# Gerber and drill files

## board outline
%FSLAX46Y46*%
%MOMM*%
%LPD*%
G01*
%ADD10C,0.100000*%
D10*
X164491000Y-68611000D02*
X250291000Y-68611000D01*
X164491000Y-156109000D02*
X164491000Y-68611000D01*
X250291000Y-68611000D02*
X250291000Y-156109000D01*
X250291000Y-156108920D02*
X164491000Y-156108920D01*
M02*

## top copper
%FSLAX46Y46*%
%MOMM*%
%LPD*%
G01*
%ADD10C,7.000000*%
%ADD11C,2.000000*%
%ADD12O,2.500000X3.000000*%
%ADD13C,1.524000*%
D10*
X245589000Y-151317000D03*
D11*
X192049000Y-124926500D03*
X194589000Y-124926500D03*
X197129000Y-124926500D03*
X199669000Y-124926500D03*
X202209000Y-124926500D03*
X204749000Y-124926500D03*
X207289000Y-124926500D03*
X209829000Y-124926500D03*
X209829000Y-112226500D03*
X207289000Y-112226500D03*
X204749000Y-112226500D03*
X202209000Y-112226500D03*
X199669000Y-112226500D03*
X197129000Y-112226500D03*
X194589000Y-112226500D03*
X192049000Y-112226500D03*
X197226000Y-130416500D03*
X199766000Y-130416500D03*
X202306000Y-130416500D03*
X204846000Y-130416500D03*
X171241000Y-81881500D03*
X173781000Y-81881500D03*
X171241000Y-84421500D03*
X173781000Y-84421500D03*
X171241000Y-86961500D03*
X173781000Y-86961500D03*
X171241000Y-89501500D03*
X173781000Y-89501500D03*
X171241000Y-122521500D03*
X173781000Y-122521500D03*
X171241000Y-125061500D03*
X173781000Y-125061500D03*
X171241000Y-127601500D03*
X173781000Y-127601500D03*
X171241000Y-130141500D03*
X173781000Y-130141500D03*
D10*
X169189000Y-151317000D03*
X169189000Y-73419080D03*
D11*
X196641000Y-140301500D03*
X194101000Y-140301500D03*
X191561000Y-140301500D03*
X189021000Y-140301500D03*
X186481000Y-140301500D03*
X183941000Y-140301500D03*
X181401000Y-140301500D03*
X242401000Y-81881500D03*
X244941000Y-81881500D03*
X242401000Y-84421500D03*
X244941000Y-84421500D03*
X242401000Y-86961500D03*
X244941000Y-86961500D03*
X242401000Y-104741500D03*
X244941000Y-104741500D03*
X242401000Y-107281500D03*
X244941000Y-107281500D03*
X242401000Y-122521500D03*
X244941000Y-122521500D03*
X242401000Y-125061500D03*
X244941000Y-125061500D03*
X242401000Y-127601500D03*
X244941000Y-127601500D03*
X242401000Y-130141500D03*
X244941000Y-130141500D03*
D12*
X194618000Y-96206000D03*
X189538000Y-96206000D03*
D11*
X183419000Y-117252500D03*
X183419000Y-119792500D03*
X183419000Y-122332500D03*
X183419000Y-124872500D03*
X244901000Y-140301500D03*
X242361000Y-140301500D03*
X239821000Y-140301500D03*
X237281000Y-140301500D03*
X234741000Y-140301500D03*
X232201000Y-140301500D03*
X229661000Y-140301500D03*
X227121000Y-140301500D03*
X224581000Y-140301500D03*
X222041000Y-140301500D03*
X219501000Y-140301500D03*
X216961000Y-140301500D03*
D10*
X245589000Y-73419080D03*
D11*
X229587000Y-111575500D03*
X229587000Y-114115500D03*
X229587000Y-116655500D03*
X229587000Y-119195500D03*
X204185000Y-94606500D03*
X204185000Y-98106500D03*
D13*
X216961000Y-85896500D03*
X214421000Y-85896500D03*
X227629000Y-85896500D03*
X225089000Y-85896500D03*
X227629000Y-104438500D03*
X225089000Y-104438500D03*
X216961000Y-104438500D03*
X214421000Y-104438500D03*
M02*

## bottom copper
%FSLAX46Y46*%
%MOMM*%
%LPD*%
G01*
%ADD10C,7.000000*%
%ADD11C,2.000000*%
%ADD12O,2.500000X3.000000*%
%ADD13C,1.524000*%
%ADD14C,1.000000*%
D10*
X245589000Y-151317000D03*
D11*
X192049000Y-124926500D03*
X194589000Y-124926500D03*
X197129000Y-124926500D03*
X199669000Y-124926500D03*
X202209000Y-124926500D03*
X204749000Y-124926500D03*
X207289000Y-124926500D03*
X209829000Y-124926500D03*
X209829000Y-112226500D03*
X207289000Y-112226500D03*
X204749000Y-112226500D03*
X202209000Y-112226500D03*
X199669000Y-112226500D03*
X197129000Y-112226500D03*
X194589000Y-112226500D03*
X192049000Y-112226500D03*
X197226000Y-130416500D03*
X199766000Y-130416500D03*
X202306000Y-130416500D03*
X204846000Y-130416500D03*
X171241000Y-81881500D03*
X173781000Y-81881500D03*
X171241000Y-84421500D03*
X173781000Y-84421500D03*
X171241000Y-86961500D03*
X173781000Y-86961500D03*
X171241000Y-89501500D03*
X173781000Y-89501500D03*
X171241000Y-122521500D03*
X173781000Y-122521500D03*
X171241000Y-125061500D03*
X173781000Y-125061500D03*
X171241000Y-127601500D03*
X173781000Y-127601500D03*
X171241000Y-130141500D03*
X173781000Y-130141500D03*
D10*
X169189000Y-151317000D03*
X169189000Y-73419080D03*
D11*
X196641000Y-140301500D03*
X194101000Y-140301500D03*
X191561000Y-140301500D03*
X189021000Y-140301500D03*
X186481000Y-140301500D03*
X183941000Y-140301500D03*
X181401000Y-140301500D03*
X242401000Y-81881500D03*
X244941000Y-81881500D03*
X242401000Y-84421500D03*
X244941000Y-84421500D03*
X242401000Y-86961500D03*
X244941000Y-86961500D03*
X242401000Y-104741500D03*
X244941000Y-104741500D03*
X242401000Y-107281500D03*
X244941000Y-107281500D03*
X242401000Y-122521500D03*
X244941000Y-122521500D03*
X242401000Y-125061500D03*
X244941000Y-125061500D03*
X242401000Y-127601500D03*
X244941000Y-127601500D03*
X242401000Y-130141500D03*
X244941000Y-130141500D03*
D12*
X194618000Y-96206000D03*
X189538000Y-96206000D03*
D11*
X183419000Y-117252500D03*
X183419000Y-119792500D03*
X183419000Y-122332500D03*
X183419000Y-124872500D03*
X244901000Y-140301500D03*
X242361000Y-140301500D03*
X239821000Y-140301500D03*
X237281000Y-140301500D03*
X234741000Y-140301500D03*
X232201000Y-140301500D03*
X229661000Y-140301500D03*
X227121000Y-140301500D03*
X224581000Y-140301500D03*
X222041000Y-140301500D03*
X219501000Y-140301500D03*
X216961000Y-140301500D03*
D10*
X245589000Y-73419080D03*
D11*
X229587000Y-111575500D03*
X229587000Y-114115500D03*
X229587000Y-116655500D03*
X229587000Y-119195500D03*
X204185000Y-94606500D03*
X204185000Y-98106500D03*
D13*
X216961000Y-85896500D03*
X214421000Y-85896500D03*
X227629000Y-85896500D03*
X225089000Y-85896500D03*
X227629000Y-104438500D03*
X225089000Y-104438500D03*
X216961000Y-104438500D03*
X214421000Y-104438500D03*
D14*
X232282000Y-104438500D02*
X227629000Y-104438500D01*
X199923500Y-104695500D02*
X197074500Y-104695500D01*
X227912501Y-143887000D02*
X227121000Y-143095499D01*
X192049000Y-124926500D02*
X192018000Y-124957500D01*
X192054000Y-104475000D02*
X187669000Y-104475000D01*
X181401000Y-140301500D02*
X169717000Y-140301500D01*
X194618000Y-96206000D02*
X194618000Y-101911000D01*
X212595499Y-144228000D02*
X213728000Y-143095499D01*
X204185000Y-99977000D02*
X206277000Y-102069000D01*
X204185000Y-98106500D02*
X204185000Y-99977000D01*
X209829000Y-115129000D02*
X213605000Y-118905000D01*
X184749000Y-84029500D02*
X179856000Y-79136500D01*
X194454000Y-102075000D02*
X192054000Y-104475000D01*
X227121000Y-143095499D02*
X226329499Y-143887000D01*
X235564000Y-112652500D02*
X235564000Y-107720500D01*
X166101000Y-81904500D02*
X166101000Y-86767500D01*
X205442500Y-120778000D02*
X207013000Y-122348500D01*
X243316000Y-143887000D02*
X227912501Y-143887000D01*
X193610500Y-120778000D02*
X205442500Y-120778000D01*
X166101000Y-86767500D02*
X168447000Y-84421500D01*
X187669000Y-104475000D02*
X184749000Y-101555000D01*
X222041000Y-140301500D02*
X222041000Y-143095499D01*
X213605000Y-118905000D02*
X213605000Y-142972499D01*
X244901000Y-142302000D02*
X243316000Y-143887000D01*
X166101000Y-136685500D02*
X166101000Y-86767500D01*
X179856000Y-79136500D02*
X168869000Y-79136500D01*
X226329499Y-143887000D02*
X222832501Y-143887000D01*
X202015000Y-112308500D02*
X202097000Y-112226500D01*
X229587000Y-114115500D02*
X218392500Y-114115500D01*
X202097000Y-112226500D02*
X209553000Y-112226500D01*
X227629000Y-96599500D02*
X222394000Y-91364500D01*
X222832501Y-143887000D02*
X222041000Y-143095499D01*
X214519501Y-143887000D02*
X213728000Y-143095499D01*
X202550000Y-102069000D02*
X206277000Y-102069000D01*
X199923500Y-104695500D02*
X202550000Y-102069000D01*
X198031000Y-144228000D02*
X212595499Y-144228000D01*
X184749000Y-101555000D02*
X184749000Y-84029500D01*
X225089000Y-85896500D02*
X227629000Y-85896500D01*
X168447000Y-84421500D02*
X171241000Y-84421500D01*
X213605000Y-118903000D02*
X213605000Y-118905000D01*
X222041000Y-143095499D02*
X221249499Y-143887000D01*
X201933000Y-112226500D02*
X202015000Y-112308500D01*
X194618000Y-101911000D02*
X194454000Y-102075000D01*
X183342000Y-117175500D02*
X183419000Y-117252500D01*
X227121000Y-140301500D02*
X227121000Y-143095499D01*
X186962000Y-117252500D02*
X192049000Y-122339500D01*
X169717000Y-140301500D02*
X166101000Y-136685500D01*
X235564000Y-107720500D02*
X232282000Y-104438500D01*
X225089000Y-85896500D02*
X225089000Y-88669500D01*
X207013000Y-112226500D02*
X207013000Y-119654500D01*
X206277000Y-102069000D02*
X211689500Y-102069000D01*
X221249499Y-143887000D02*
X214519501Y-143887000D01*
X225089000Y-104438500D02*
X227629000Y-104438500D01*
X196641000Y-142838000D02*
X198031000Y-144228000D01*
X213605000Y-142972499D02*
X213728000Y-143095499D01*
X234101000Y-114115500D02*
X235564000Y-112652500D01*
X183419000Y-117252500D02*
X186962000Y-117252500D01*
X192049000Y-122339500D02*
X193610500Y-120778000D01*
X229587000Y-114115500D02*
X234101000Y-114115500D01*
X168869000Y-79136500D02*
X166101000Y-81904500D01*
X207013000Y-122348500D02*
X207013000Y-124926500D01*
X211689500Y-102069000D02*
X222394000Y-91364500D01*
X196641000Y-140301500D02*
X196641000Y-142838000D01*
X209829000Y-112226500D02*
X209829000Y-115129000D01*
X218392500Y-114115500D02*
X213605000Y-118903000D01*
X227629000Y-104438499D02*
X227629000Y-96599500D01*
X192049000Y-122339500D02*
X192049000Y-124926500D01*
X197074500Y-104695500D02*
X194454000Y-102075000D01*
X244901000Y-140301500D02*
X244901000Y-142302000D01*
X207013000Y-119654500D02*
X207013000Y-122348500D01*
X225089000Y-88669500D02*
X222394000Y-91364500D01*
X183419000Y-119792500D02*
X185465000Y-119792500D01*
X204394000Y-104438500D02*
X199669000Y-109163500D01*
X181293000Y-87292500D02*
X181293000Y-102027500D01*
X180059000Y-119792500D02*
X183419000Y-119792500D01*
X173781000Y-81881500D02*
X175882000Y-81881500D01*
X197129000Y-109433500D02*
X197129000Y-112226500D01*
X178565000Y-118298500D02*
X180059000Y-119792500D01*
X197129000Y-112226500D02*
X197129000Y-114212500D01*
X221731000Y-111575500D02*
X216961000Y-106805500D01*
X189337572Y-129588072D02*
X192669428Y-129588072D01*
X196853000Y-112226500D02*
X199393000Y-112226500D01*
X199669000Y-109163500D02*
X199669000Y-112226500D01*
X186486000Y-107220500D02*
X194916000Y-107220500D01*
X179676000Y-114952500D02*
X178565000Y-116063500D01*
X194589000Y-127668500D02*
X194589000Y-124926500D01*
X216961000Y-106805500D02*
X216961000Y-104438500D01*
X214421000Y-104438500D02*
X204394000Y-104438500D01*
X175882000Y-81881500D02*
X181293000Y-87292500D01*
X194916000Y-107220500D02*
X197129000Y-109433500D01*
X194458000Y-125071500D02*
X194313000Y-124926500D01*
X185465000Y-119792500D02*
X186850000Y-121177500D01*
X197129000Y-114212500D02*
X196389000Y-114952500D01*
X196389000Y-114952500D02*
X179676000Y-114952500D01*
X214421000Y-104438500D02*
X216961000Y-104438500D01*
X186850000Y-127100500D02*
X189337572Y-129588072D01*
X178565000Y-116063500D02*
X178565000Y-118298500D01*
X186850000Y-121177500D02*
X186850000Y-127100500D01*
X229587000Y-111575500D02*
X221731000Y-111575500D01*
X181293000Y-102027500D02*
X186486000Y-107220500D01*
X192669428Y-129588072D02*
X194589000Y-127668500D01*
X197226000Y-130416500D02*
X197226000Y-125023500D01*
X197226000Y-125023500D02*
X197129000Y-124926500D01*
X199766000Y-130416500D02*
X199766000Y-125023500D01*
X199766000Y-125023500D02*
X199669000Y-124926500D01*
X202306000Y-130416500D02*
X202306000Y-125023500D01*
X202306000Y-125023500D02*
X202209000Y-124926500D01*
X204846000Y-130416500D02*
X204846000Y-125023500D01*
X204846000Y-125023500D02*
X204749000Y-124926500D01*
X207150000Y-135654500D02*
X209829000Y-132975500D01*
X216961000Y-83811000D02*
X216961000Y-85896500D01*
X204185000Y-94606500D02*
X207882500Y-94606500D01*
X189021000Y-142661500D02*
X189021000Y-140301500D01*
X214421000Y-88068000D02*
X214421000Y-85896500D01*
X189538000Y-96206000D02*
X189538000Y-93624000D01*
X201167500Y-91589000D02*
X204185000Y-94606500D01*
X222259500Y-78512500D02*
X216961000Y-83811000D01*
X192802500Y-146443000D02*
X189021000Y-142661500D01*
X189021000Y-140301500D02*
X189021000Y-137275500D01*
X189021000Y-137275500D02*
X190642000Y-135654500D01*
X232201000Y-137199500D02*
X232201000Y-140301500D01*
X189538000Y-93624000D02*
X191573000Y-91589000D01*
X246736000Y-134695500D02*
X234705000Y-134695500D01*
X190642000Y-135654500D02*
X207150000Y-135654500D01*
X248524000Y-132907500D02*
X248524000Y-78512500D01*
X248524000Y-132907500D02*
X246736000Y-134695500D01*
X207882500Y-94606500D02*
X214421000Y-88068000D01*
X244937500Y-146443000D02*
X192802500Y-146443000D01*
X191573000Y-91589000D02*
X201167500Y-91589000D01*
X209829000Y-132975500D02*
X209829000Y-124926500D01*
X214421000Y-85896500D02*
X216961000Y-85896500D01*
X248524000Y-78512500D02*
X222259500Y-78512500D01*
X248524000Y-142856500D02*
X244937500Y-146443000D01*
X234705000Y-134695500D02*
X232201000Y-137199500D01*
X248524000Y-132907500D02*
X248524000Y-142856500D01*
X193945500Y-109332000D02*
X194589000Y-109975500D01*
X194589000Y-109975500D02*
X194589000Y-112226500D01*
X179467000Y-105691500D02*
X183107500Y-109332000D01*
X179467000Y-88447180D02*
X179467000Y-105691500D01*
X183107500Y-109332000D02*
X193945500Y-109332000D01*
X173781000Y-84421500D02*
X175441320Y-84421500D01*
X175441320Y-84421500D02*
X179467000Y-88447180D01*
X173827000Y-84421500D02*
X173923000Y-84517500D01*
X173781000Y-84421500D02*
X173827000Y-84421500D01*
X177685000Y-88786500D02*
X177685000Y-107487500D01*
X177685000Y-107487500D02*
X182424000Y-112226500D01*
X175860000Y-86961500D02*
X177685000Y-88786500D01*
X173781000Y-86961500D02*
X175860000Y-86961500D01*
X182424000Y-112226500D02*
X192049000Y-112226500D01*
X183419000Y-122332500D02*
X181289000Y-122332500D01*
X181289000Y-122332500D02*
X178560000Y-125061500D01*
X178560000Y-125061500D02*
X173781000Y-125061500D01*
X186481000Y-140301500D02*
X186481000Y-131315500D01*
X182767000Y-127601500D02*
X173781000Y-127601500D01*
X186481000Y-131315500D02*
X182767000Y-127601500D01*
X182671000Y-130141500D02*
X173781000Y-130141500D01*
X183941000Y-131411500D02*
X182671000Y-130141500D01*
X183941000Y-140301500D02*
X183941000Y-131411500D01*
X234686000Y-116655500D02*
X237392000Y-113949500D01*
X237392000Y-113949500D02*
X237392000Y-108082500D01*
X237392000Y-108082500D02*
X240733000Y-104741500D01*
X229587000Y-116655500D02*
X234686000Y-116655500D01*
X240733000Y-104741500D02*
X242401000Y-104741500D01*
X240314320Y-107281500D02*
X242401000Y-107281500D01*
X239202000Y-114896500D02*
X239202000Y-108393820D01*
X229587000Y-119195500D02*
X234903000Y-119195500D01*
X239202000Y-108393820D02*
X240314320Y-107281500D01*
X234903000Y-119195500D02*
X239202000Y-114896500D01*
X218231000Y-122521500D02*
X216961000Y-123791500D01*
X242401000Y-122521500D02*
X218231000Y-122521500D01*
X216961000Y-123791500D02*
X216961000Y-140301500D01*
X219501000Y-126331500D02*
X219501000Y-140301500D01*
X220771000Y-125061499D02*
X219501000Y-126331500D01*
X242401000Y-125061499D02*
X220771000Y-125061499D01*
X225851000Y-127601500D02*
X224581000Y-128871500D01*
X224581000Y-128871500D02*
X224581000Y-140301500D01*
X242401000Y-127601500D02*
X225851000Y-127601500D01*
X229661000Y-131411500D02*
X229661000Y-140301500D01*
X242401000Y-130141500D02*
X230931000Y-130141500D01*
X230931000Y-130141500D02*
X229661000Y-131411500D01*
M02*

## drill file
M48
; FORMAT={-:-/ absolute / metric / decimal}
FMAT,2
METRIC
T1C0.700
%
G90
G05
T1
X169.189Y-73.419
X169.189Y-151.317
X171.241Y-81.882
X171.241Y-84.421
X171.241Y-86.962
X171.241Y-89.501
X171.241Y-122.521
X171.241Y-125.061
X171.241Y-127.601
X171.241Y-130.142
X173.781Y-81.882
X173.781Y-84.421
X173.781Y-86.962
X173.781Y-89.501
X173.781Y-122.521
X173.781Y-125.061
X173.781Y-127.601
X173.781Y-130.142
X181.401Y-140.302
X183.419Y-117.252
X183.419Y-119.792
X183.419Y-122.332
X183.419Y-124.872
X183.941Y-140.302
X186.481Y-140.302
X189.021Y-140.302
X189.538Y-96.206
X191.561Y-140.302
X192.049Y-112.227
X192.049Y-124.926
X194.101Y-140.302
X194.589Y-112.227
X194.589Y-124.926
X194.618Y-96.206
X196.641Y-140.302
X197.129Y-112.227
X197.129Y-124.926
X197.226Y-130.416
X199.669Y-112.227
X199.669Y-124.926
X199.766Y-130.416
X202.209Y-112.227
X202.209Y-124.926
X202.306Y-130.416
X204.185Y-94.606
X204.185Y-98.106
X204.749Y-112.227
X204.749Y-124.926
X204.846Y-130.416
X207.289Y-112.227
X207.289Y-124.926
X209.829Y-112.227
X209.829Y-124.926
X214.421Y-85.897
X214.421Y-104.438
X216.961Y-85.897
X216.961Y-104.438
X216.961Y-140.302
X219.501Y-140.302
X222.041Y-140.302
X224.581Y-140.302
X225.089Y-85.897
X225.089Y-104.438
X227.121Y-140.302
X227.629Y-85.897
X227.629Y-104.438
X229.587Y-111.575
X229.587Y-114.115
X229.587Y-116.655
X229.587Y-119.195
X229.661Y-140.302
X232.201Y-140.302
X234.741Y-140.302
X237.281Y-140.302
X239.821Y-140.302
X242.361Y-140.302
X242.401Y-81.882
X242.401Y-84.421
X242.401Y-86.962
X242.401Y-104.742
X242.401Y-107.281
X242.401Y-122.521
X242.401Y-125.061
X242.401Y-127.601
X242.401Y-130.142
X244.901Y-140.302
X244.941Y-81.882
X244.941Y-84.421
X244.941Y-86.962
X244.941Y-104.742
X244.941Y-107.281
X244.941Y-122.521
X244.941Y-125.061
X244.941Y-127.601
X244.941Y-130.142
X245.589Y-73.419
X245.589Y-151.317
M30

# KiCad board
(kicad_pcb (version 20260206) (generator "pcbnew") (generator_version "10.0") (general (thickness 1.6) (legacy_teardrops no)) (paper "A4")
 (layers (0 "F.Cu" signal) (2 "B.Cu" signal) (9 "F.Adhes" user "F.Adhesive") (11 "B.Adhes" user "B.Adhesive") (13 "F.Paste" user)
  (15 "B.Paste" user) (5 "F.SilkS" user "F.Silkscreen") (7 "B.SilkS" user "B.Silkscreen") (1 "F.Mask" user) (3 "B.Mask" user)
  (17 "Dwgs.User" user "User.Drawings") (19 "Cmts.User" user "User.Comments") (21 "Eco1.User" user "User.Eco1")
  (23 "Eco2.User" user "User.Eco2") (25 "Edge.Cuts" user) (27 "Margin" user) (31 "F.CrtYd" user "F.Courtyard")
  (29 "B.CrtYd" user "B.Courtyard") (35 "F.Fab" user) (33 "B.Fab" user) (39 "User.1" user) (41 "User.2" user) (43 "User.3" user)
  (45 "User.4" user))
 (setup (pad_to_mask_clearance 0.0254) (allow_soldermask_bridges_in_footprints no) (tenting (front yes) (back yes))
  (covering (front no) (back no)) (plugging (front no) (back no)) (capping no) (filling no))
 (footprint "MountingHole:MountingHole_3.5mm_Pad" (layer "F.Cu") (at 245.589 151.317)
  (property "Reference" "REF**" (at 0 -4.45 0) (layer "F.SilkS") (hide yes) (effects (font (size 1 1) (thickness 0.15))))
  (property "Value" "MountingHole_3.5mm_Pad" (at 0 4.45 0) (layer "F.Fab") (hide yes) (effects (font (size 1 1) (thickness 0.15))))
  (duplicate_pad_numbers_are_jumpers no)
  (pad "1" thru_hole circle (at 0 0) (size 7 7) (drill 0.7) (layers "*.Cu" "*.Mask") (remove_unused_layers no) (zone_connect 2)))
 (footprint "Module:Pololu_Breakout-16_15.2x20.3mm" (layer "F.Cu") (at 192.049 124.9265 90)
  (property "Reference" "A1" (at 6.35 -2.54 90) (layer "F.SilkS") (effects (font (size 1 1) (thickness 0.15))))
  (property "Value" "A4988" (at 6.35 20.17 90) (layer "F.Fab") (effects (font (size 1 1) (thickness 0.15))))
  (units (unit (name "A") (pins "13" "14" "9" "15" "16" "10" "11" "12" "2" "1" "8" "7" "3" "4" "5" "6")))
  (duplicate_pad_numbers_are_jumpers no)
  (pad "1" thru_hole circle (at 0 0 90) (size 2 2) (drill 0.7) (layers "*.Cu" "*.Mask") (remove_unused_layers no) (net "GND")
   (thermal_bridge_angle 90))
  (pad "2" thru_hole circle (at 0 2.54 90) (size 2 2) (drill 0.7) (layers "*.Cu" "*.Mask") (remove_unused_layers no) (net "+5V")
   (thermal_bridge_angle 90))
  (pad "3" thru_hole circle (at 0 5.08 90) (size 2 2) (drill 0.7) (layers "*.Cu" "*.Mask") (remove_unused_layers no) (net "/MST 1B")
   (thermal_bridge_angle 90))
  (pad "4" thru_hole circle (at 0 7.62 90) (size 2 2) (drill 0.7) (layers "*.Cu" "*.Mask") (remove_unused_layers no) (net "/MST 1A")
   (thermal_bridge_angle 90))
  (pad "5" thru_hole circle (at 0 10.16 90) (size 2 2) (drill 0.7) (layers "*.Cu" "*.Mask") (remove_unused_layers no) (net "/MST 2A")
   (thermal_bridge_angle 90))
  (pad "6" thru_hole circle (at 0 12.7 90) (size 2 2) (drill 0.7) (layers "*.Cu" "*.Mask") (remove_unused_layers no) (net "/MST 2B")
   (thermal_bridge_angle 90))
  (pad "7" thru_hole circle (at 0 15.24 90) (size 2 2) (drill 0.7) (layers "*.Cu" "*.Mask") (remove_unused_layers no) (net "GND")
   (thermal_bridge_angle 90))
  (pad "8" thru_hole circle (at 0 17.78 90) (size 2 2) (drill 0.7) (layers "*.Cu" "*.Mask") (remove_unused_layers no) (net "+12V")
   (thermal_bridge_angle 90))
  (pad "9" thru_hole circle (at 12.7 17.78 90) (size 2 2) (drill 0.7) (layers "*.Cu" "*.Mask") (remove_unused_layers no) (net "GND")
   (thermal_bridge_angle 90))
  (pad "10" thru_hole circle (at 12.7 15.24 90) (size 2 2) (drill 0.7) (layers "*.Cu" "*.Mask") (remove_unused_layers no) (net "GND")
   (thermal_bridge_angle 90))
  (pad "11" thru_hole circle (at 12.7 12.7 90) (size 2 2) (drill 0.7) (layers "*.Cu" "*.Mask") (remove_unused_layers no) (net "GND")
   (thermal_bridge_angle 90))
  (pad "12" thru_hole circle (at 12.7 10.16 90) (size 2 2) (drill 0.7) (layers "*.Cu" "*.Mask") (remove_unused_layers no) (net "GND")
   (thermal_bridge_angle 90))
  (pad "13" thru_hole circle (at 12.7 7.62 90) (size 2 2) (drill 0.7) (layers "*.Cu" "*.Mask") (remove_unused_layers no) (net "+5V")
   (thermal_bridge_angle 90))
  (pad "14" thru_hole circle (at 12.7 5.08 90) (size 2 2) (drill 0.7) (layers "*.Cu" "*.Mask") (remove_unused_layers no) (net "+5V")
   (thermal_bridge_angle 90))
  (pad "15" thru_hole circle (at 12.7 2.54 90) (size 2 2) (drill 0.7) (layers "*.Cu" "*.Mask") (remove_unused_layers no) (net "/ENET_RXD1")
   (thermal_bridge_angle 90))
  (pad "16" thru_hole circle (at 12.7 0 90) (size 2 2) (drill 0.7) (layers "*.Cu" "*.Mask") (remove_unused_layers no) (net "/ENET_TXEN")
   (thermal_bridge_angle 90)))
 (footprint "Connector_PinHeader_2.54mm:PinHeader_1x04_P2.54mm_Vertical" (layer "F.Cu") (at 197.226 130.4165 90)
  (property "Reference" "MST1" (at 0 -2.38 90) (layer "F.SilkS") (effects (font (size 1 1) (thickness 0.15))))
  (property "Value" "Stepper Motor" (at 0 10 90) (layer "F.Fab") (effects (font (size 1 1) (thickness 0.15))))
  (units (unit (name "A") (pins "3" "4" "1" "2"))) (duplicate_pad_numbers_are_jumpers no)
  (pad "1" thru_hole circle (at 0 0 90) (size 2 2) (drill 0.7) (layers "*.Cu" "*.Mask") (remove_unused_layers no) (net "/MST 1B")
   (thermal_bridge_angle 90))
  (pad "2" thru_hole circle (at 0 2.54 90) (size 2 2) (drill 0.7) (layers "*.Cu" "*.Mask") (remove_unused_layers no) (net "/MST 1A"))
  (pad "3" thru_hole circle (at 0 5.08 90) (size 2 2) (drill 0.7) (layers "*.Cu" "*.Mask") (remove_unused_layers no) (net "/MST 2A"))
  (pad "4" thru_hole circle (at 0 7.62 90) (size 2 2) (drill 0.7) (layers "*.Cu" "*.Mask") (remove_unused_layers no) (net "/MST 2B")))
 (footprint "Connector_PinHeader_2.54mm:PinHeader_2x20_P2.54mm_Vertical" (layer "F.Cu") (at 171.241 81.8815)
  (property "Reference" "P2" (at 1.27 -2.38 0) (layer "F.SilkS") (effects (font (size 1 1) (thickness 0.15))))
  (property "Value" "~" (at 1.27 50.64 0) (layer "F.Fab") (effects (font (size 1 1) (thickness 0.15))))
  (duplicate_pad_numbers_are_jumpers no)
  (pad "1" thru_hole circle (at 0 0) (size 2 2) (drill 0.7) (layers "*.Cu" "*.Mask") (remove_unused_layers no)
   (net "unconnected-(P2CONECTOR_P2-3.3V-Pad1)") (thermal_bridge_angle 90))
  (pad "2" thru_hole circle (at 2.54 0) (size 2 2) (drill 0.7) (layers "*.Cu" "*.Mask") (remove_unused_layers no) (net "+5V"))
  (pad "3" thru_hole circle (at 0 2.54) (size 2 2) (drill 0.7) (layers "*.Cu" "*.Mask") (remove_unused_layers no) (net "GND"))
  (pad "4" thru_hole circle (at 2.54 2.54) (size 2 2) (drill 0.7) (layers "*.Cu" "*.Mask") (remove_unused_layers no) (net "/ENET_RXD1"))
  (pad "5" thru_hole circle (at 0 5.08) (size 2 2) (drill 0.7) (layers "*.Cu" "*.Mask") (remove_unused_layers no)
   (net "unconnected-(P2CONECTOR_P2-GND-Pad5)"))
  (pad "6" thru_hole circle (at 2.54 5.08) (size 2 2) (drill 0.7) (layers "*.Cu" "*.Mask") (remove_unused_layers no) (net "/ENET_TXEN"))
  (pad "7" thru_hole circle (at 0 7.62) (size 2 2) (drill 0.7) (layers "*.Cu" "*.Mask") (remove_unused_layers no)
   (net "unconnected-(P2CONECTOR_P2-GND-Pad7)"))
  (pad "8" thru_hole circle (at 2.54 7.62) (size 2 2) (drill 0.7) (layers "*.Cu" "*.Mask") (remove_unused_layers no)
   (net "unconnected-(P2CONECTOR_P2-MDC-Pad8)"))
  (pad "33" thru_hole circle (at 0 40.64) (size 2 2) (drill 0.7) (layers "*.Cu" "*.Mask") (remove_unused_layers no)
   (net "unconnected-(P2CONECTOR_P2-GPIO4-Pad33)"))
  (pad "34" thru_hole circle (at 2.54 40.64) (size 2 2) (drill 0.7) (layers "*.Cu" "*.Mask") (remove_unused_layers no)
   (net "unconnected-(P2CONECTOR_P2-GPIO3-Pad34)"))
  (pad "35" thru_hole circle (at 0 43.18) (size 2 2) (drill 0.7) (layers "*.Cu" "*.Mask") (remove_unused_layers no)
   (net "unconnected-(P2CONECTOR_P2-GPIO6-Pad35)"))
  (pad "36" thru_hole circle (at 2.54 43.18) (size 2 2) (drill 0.7) (layers "*.Cu" "*.Mask") (remove_unused_layers no) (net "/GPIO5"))
  (pad "37" thru_hole circle (at 0 45.72) (size 2 2) (drill 0.7) (layers "*.Cu" "*.Mask") (remove_unused_layers no)
   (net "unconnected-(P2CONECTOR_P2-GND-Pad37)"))
  (pad "38" thru_hole circle (at 2.54 45.72) (size 2 2) (drill 0.7) (layers "*.Cu" "*.Mask") (remove_unused_layers no) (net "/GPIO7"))
  (pad "39" thru_hole circle (at 0 48.26) (size 2 2) (drill 0.7) (layers "*.Cu" "*.Mask") (remove_unused_layers no)
   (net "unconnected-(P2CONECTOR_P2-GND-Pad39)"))
  (pad "40" thru_hole circle (at 2.54 48.26) (size 2 2) (drill 0.7) (layers "*.Cu" "*.Mask") (remove_unused_layers no) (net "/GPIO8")))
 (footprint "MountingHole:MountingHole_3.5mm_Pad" (layer "F.Cu") (at 169.189 151.317)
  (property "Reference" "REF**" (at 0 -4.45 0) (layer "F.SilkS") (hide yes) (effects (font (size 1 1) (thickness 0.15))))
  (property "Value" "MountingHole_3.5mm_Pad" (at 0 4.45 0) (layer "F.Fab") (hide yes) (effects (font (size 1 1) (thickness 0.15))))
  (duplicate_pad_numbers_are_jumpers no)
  (pad "1" thru_hole circle (at 0 0) (size 7 7) (drill 0.7) (layers "*.Cu" "*.Mask") (remove_unused_layers no) (zone_connect 2)))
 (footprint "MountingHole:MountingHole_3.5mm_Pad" (layer "F.Cu") (at 169.189 73.41908)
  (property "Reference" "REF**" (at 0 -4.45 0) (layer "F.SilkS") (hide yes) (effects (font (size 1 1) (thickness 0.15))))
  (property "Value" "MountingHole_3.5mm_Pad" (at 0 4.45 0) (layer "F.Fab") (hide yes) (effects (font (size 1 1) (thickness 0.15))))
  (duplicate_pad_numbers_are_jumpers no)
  (pad "1" thru_hole circle (at 0 0) (size 7 7) (drill 0.7) (layers "*.Cu" "*.Mask") (remove_unused_layers no) (zone_connect 2)))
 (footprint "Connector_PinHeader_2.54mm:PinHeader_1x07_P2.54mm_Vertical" (layer "F.Cu") (at 196.641 140.3015 -90)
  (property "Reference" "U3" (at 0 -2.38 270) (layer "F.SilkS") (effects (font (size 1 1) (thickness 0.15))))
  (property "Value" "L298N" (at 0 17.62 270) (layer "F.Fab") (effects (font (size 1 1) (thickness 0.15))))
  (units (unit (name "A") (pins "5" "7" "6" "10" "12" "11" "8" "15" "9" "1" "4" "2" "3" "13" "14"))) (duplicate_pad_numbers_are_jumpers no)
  (pad "1" thru_hole circle (at 0 0 270) (size 2 2) (drill 0.7) (layers "*.Cu" "*.Mask") (remove_unused_layers no) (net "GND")
   (thermal_bridge_angle 90))
  (pad "2" thru_hole circle (at 0 2.54 270) (size 2 2) (drill 0.7) (layers "*.Cu" "*.Mask") (remove_unused_layers no) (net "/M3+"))
  (pad "3" thru_hole circle (at 0 5.08 270) (size 2 2) (drill 0.7) (layers "*.Cu" "*.Mask") (remove_unused_layers no) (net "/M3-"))
  (pad "4" thru_hole circle (at 0 7.62 270) (size 2 2) (drill 0.7) (layers "*.Cu" "*.Mask") (remove_unused_layers no) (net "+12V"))
  (pad "5" thru_hole circle (at 0 10.16 270) (size 2 2) (drill 0.7) (layers "*.Cu" "*.Mask") (remove_unused_layers no) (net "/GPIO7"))
  (pad "6" thru_hole circle (at 0 12.7 270) (size 2 2) (drill 0.7) (layers "*.Cu" "*.Mask") (remove_unused_layers no) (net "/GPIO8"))
  (pad "7" thru_hole circle (at 0 15.24 270) (size 2 2) (drill 0.7) (layers "*.Cu" "*.Mask") (remove_unused_layers no) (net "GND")))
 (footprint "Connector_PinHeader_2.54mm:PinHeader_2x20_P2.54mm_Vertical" (layer "F.Cu") (at 242.401 81.8815)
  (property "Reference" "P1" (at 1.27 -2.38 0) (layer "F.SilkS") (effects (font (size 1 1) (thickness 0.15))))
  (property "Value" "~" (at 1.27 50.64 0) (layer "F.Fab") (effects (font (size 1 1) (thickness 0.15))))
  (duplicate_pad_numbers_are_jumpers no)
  (pad "1" thru_hole circle (at 0 0) (size 2 2) (drill 0.7) (layers "*.Cu" "*.Mask") (remove_unused_layers no)
   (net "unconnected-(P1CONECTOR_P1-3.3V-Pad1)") (thermal_bridge_angle 90))
  (pad "2" thru_hole circle (at 2.54 0) (size 2 2) (drill 0.7) (layers "*.Cu" "*.Mask") (remove_unused_layers no)
   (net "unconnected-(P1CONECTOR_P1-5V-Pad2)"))
  (pad "3" thru_hole circle (at 0 2.54) (size 2 2) (drill 0.7) (layers "*.Cu" "*.Mask") (remove_unused_layers no)
   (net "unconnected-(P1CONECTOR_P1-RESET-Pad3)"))
  (pad "4" thru_hole circle (at 2.54 2.54) (size 2 2) (drill 0.7) (layers "*.Cu" "*.Mask") (remove_unused_layers no)
   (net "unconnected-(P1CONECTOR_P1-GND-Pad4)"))
  (pad "5" thru_hole circle (at 0 5.08) (size 2 2) (drill 0.7) (layers "*.Cu" "*.Mask") (remove_unused_layers no)
   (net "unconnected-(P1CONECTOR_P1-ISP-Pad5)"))
  (pad "6" thru_hole circle (at 2.54 5.08) (size 2 2) (drill 0.7) (layers "*.Cu" "*.Mask") (remove_unused_layers no)
   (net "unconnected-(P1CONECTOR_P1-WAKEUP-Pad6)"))
  (pad "19" thru_hole circle (at 0 22.86) (size 2 2) (drill 0.7) (layers "*.Cu" "*.Mask") (remove_unused_layers no) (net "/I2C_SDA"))
  (pad "20" thru_hole circle (at 2.54 22.86) (size 2 2) (drill 0.7) (layers "*.Cu" "*.Mask") (remove_unused_layers no)
   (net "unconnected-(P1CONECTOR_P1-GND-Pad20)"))
  (pad "21" thru_hole circle (at 0 25.4) (size 2 2) (drill 0.7) (layers "*.Cu" "*.Mask") (remove_unused_layers no) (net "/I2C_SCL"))
  (pad "22" thru_hole circle (at 2.54 25.4) (size 2 2) (drill 0.7) (layers "*.Cu" "*.Mask") (remove_unused_layers no)
   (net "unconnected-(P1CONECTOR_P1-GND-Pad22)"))
  (pad "33" thru_hole circle (at 0 40.64) (size 2 2) (drill 0.7) (layers "*.Cu" "*.Mask") (remove_unused_layers no) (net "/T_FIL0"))
  (pad "34" thru_hole circle (at 2.54 40.64) (size 2 2) (drill 0.7) (layers "*.Cu" "*.Mask") (remove_unused_layers no)
   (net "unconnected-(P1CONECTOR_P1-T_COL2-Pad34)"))
  (pad "35" thru_hole circle (at 0 43.18) (size 2 2) (drill 0.7) (layers "*.Cu" "*.Mask") (remove_unused_layers no) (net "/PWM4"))
  (pad "36" thru_hole circle (at 2.54 43.18) (size 2 2) (drill 0.7) (layers "*.Cu" "*.Mask") (remove_unused_layers no)
   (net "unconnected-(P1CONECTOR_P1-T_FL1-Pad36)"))
  (pad "37" thru_hole circle (at 0 45.72) (size 2 2) (drill 0.7) (layers "*.Cu" "*.Mask") (remove_unused_layers no) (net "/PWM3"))
  (pad "38" thru_hole circle (at 2.54 45.72) (size 2 2) (drill 0.7) (layers "*.Cu" "*.Mask") (remove_unused_layers no)
   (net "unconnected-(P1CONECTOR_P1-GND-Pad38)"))
  (pad "39" thru_hole circle (at 0 48.26) (size 2 2) (drill 0.7) (layers "*.Cu" "*.Mask") (remove_unused_layers no) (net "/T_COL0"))
  (pad "40" thru_hole circle (at 2.54 48.26) (size 2 2) (drill 0.7) (layers "*.Cu" "*.Mask") (remove_unused_layers no)
   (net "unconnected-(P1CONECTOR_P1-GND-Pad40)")))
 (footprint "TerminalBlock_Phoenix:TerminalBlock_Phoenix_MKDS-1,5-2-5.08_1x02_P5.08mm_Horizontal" (layer "F.Cu") (at 194.618 96.206 180)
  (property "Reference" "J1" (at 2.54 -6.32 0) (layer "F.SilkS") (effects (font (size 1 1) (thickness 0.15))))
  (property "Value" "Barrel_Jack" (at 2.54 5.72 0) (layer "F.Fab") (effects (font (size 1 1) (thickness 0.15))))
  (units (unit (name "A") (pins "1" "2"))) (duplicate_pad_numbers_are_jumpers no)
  (pad "1" thru_hole oval (at 0 0 180) (size 2.5 3) (drill 0.7) (layers "*.Cu" "*.Mask") (remove_unused_layers no) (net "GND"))
  (pad "2" thru_hole oval (at 5.08 0 180) (size 2.5 3) (drill 0.7) (layers "*.Cu" "*.Mask") (remove_unused_layers no) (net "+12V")
   (thermal_bridge_angle 45)))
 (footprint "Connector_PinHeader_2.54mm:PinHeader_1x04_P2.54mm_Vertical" (layer "F.Cu") (at 183.419 117.2525)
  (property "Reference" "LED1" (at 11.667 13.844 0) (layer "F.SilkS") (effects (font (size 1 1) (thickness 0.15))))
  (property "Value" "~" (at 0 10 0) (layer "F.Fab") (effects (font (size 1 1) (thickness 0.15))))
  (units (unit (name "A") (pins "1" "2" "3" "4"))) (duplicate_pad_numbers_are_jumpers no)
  (pad "1" thru_hole circle (at 0 0) (size 2 2) (drill 0.7) (layers "*.Cu" "*.Mask") (remove_unused_layers no) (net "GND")
   (thermal_bridge_angle 90))
  (pad "2" thru_hole circle (at 0 2.54) (size 2 2) (drill 0.7) (layers "*.Cu" "*.Mask") (remove_unused_layers no) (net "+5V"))
  (pad "3" thru_hole circle (at 0 5.08) (size 2 2) (drill 0.7) (layers "*.Cu" "*.Mask") (remove_unused_layers no) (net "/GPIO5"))
  (pad "4" thru_hole circle (at 0 7.62) (size 2 2) (drill 0.7) (layers "*.Cu" "*.Mask") (remove_unused_layers no)
   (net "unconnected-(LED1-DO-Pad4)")))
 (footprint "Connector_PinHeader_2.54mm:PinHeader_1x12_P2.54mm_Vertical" (layer "F.Cu") (at 244.901 140.3015 -90)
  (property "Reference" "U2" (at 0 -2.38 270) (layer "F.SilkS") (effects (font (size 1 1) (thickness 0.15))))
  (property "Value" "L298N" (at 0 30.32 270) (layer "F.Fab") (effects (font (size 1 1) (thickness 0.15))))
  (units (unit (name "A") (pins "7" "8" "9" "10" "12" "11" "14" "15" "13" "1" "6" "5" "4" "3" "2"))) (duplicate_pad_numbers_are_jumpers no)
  (pad "1" thru_hole circle (at 0 0 270) (size 2 2) (drill 0.7) (layers "*.Cu" "*.Mask") (remove_unused_layers no) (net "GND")
   (thermal_bridge_angle 90))
  (pad "2" thru_hole circle (at 0 2.54 270) (size 2 2) (drill 0.7) (layers "*.Cu" "*.Mask") (remove_unused_layers no) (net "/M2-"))
  (pad "3" thru_hole circle (at 0 5.08 270) (size 2 2) (drill 0.7) (layers "*.Cu" "*.Mask") (remove_unused_layers no) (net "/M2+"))
  (pad "4" thru_hole circle (at 0 7.62 270) (size 2 2) (drill 0.7) (layers "*.Cu" "*.Mask") (remove_unused_layers no) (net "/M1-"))
  (pad "5" thru_hole circle (at 0 10.16 270) (size 2 2) (drill 0.7) (layers "*.Cu" "*.Mask") (remove_unused_layers no) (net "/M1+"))
  (pad "6" thru_hole circle (at 0 12.7 270) (size 2 2) (drill 0.7) (layers "*.Cu" "*.Mask") (remove_unused_layers no) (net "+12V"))
  (pad "7" thru_hole circle (at 0 15.24 270) (size 2 2) (drill 0.7) (layers "*.Cu" "*.Mask") (remove_unused_layers no) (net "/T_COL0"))
  (pad "8" thru_hole circle (at 0 17.78 270) (size 2 2) (drill 0.7) (layers "*.Cu" "*.Mask") (remove_unused_layers no) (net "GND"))
  (pad "9" thru_hole circle (at 0 20.32 270) (size 2 2) (drill 0.7) (layers "*.Cu" "*.Mask") (remove_unused_layers no) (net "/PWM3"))
  (pad "10" thru_hole circle (at 0 22.86 270) (size 2 2) (drill 0.7) (layers "*.Cu" "*.Mask") (remove_unused_layers no) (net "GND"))
  (pad "11" thru_hole circle (at 0 25.4 270) (size 2 2) (drill 0.7) (layers "*.Cu" "*.Mask") (remove_unused_layers no) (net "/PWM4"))
  (pad "12" thru_hole circle (at 0 27.94 270) (size 2 2) (drill 0.7) (layers "*.Cu" "*.Mask") (remove_unused_layers no) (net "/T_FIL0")))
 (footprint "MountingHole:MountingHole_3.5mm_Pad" (layer "F.Cu") (at 245.589 73.41908)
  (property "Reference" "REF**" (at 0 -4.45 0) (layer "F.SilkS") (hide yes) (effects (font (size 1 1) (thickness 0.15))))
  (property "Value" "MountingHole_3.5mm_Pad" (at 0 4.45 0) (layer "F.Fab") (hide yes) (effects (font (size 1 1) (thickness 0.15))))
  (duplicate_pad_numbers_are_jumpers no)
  (pad "1" thru_hole circle (at 0 0) (size 7 7) (drill 0.7) (layers "*.Cu" "*.Mask") (remove_unused_layers no) (zone_connect 2)))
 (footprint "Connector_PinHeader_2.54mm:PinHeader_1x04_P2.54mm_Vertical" (layer "F.Cu") (at 229.587 111.5755)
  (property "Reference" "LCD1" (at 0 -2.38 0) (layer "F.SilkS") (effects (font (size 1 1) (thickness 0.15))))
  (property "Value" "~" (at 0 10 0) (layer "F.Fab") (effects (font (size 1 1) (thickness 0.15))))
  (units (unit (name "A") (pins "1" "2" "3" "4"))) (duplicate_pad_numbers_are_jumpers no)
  (pad "1" thru_hole circle (at 0 0) (size 2 2) (drill 0.7) (layers "*.Cu" "*.Mask") (remove_unused_layers no) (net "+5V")
   (thermal_bridge_angle 90))
  (pad "2" thru_hole circle (at 0 2.54) (size 2 2) (drill 0.7) (layers "*.Cu" "*.Mask") (remove_unused_layers no) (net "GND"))
  (pad "3" thru_hole circle (at 0 5.08) (size 2 2) (drill 0.7) (layers "*.Cu" "*.Mask") (remove_unused_layers no) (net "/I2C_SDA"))
  (pad "4" thru_hole circle (at 0 7.62) (size 2 2) (drill 0.7) (layers "*.Cu" "*.Mask") (remove_unused_layers no) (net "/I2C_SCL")))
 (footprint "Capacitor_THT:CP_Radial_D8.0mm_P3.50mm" (layer "F.Cu") (at 204.185 94.6065 -90)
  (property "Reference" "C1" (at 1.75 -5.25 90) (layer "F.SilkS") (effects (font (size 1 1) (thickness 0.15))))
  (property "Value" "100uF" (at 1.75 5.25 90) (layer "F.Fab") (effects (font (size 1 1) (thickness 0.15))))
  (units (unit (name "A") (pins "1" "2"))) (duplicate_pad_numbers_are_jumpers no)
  (pad "1" thru_hole circle (at 0 0 270) (size 2 2) (drill 0.7) (layers "*.Cu" "*.Mask") (remove_unused_layers no) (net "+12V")
   (thermal_bridge_angle 90))
  (pad "2" thru_hole circle (at 3.5 0 270) (size 2 2) (drill 0.7) (layers "*.Cu" "*.Mask") (remove_unused_layers no) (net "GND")))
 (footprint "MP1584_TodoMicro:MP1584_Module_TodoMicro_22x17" (layer "F.Cu") (at 221.025 95.1675 -90)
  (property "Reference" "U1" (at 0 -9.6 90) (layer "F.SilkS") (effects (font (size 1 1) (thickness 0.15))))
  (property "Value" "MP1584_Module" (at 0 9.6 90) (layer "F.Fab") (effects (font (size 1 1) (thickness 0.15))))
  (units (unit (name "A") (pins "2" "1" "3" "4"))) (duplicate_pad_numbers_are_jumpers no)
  (pad "1" thru_hole circle (at -9.271 4.064 270) (size 1.524 1.524) (drill 0.7) (layers "*.Cu" "*.Mask") (remove_unused_layers no)
   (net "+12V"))
  (pad "1" thru_hole circle (at -9.271 6.604 270) (size 1.524 1.524) (drill 0.7) (layers "*.Cu" "*.Mask") (remove_unused_layers no)
   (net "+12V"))
  (pad "2" thru_hole circle (at -9.271 -6.604 270) (size 1.524 1.524) (drill 0.7) (layers "*.Cu" "*.Mask") (remove_unused_layers no)
   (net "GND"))
  (pad "2" thru_hole circle (at -9.271 -4.064 270) (size 1.524 1.524) (drill 0.7) (layers "*.Cu" "*.Mask") (remove_unused_layers no)
   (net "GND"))
  (pad "3" thru_hole circle (at 9.271 -6.604 270) (size 1.524 1.524) (drill 0.7) (layers "*.Cu" "*.Mask") (remove_unused_layers no)
   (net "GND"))
  (pad "3" thru_hole circle (at 9.271 -4.064 270) (size 1.524 1.524) (drill 0.7) (layers "*.Cu" "*.Mask") (remove_unused_layers no)
   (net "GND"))
  (pad "4" thru_hole circle (at 9.271 4.064 270) (size 1.524 1.524) (drill 0.7) (layers "*.Cu" "*.Mask") (remove_unused_layers no)
   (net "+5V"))
  (pad "4" thru_hole circle (at 9.271 6.604 270) (size 1.524 1.524) (drill 0.7) (layers "*.Cu" "*.Mask") (remove_unused_layers no)
   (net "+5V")))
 (gr_line (start 164.491 68.611) (end 250.291 68.611) (stroke (width 0.1) (type default)) (layer "Edge.Cuts"))
 (gr_line (start 164.491 156.109) (end 164.491 68.611) (stroke (width 0.1) (type default)) (layer "Edge.Cuts"))
 (gr_line (start 250.291 68.611) (end 250.291 156.109) (stroke (width 0.1) (type default)) (layer "Edge.Cuts"))
 (gr_line (start 250.291 156.10892) (end 164.491 156.10892) (stroke (width 0.1) (type default)) (layer "Edge.Cuts"))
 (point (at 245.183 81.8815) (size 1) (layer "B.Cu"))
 (segment (start 232.282 104.4385) (end 227.629 104.4385) (width 1) (layer "B.Cu") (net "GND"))
 (segment (start 199.9235 104.6955) (end 197.0745 104.6955) (width 1) (layer "B.Cu") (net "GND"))
 (segment (start 227.912501 143.887) (end 227.121 143.095499) (width 1) (layer "B.Cu") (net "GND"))
 (segment (start 192.049 124.9265) (end 192.018 124.9575) (width 1) (layer "B.Cu") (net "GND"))
 (segment (start 192.054 104.475) (end 187.669 104.475) (width 1) (layer "B.Cu") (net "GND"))
 (segment (start 181.401 140.3015) (end 169.717 140.3015) (width 1) (layer "B.Cu") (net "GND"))
 (segment (start 194.618 96.206) (end 194.618 101.911) (width 1) (layer "B.Cu") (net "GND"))
 (segment (start 212.595499 144.228) (end 213.728 143.095499) (width 1) (layer "B.Cu") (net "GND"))
 (segment (start 204.185 99.977) (end 206.277 102.069) (width 1) (layer "B.Cu") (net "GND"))
 (segment (start 204.185 98.1065) (end 204.185 99.977) (width 1) (layer "B.Cu") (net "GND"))
 (segment (start 209.829 115.129) (end 213.605 118.905) (width 1) (layer "B.Cu") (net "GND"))
 (segment (start 184.749 84.0295) (end 179.856 79.1365) (width 1) (layer "B.Cu") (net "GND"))
 (segment (start 194.454 102.075) (end 192.054 104.475) (width 1) (layer "B.Cu") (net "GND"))
 (segment (start 227.121 143.095499) (end 226.329499 143.887) (width 1) (layer "B.Cu") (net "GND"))
 (segment (start 235.564 112.6525) (end 235.564 107.7205) (width 1) (layer "B.Cu") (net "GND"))
 (segment (start 166.101 81.9045) (end 166.101 86.7675) (width 1) (layer "B.Cu") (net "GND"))
 (segment (start 205.4425 120.778) (end 207.013 122.3485) (width 1) (layer "B.Cu") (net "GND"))
 (segment (start 243.316 143.887) (end 227.912501 143.887) (width 1) (layer "B.Cu") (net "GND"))
 (segment (start 193.6105 120.778) (end 205.4425 120.778) (width 1) (layer "B.Cu") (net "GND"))
 (segment (start 166.101 86.7675) (end 168.447 84.4215) (width 1) (layer "B.Cu") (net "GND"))
 (segment (start 187.669 104.475) (end 184.749 101.555) (width 1) (layer "B.Cu") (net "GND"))
 (segment (start 222.041 140.3015) (end 222.041 143.095499) (width 1) (layer "B.Cu") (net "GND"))
 (segment (start 213.605 118.905) (end 213.605 142.972499) (width 1) (layer "B.Cu") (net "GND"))
 (segment (start 244.901 142.302) (end 243.316 143.887) (width 1) (layer "B.Cu") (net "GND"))
 (segment (start 166.101 136.6855) (end 166.101 86.7675) (width 1) (layer "B.Cu") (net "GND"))
 (segment (start 179.856 79.1365) (end 168.869 79.1365) (width 1) (layer "B.Cu") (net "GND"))
 (segment (start 226.329499 143.887) (end 222.832501 143.887) (width 1) (layer "B.Cu") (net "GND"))
 (segment (start 202.015 112.3085) (end 202.097 112.2265) (width 1) (layer "B.Cu") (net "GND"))
 (segment (start 229.587 114.1155) (end 218.3925 114.1155) (width 1) (layer "B.Cu") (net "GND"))
 (segment (start 202.097 112.2265) (end 209.553 112.2265) (width 1) (layer "B.Cu") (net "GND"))
 (segment (start 227.629 96.5995) (end 222.394 91.3645) (width 1) (layer "B.Cu") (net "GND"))
 (segment (start 222.832501 143.887) (end 222.041 143.095499) (width 1) (layer "B.Cu") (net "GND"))
 (segment (start 214.519501 143.887) (end 213.728 143.095499) (width 1) (layer "B.Cu") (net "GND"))
 (segment (start 202.55 102.069) (end 206.277 102.069) (width 1) (layer "B.Cu") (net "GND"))
 (segment (start 199.9235 104.6955) (end 202.55 102.069) (width 1) (layer "B.Cu") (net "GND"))
 (segment (start 198.031 144.228) (end 212.595499 144.228) (width 1) (layer "B.Cu") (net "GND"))
 (segment (start 184.749 101.555) (end 184.749 84.0295) (width 1) (layer "B.Cu") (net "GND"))
 (segment (start 225.089 85.8965) (end 227.629 85.8965) (width 1) (layer "B.Cu") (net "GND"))
 (segment (start 168.447 84.4215) (end 171.241 84.4215) (width 1) (layer "B.Cu") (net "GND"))
 (segment (start 213.605 118.903) (end 213.605 118.905) (width 1) (layer "B.Cu") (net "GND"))
 (segment (start 222.041 143.095499) (end 221.249499 143.887) (width 1) (layer "B.Cu") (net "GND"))
 (segment (start 201.933 112.2265) (end 202.015 112.3085) (width 1) (layer "B.Cu") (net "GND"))
 (segment (start 194.618 101.911) (end 194.454 102.075) (width 1) (layer "B.Cu") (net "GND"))
 (segment (start 183.342 117.1755) (end 183.419 117.2525) (width 1) (layer "B.Cu") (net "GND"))
 (segment (start 227.121 140.3015) (end 227.121 143.095499) (width 1) (layer "B.Cu") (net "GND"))
 (segment (start 186.962 117.2525) (end 192.049 122.3395) (width 1) (layer "B.Cu") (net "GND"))
 (segment (start 169.717 140.3015) (end 166.101 136.6855) (width 1) (layer "B.Cu") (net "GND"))
 (segment (start 235.564 107.7205) (end 232.282 104.4385) (width 1) (layer "B.Cu") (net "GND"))
 (segment (start 225.089 85.8965) (end 225.089 88.6695) (width 1) (layer "B.Cu") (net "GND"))
 (segment (start 207.013 112.2265) (end 207.013 119.6545) (width 1) (layer "B.Cu") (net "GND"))
 (segment (start 206.277 102.069) (end 211.6895 102.069) (width 1) (layer "B.Cu") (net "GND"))
 (segment (start 221.249499 143.887) (end 214.519501 143.887) (width 1) (layer "B.Cu") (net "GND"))
 (segment (start 225.089 104.4385) (end 227.629 104.4385) (width 1) (layer "B.Cu") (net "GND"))
 (segment (start 196.641 142.838) (end 198.031 144.228) (width 1) (layer "B.Cu") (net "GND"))
 (segment (start 213.605 142.972499) (end 213.728 143.095499) (width 1) (layer "B.Cu") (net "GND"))
 (segment (start 234.101 114.1155) (end 235.564 112.6525) (width 1) (layer "B.Cu") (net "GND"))
 (segment (start 183.419 117.2525) (end 186.962 117.2525) (width 1) (layer "B.Cu") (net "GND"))
 (segment (start 192.049 122.3395) (end 193.6105 120.778) (width 1) (layer "B.Cu") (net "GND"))
 (segment (start 229.587 114.1155) (end 234.101 114.1155) (width 1) (layer "B.Cu") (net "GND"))
 (segment (start 168.869 79.1365) (end 166.101 81.9045) (width 1) (layer "B.Cu") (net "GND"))
 (segment (start 207.013 122.3485) (end 207.013 124.9265) (width 1) (layer "B.Cu") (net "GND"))
 (segment (start 211.6895 102.069) (end 222.394 91.3645) (width 1) (layer "B.Cu") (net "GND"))
 (segment (start 196.641 140.3015) (end 196.641 142.838) (width 1) (layer "B.Cu") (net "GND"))
 (segment (start 209.829 112.2265) (end 209.829 115.129) (width 1) (layer "B.Cu") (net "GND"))
 (segment (start 218.3925 114.1155) (end 213.605 118.903) (width 1) (layer "B.Cu") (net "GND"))
 (segment (start 227.629 104.438499) (end 227.629 96.5995) (width 1) (layer "B.Cu") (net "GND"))
 (segment (start 192.049 122.3395) (end 192.049 124.9265) (width 1) (layer "B.Cu") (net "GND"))
 (segment (start 197.0745 104.6955) (end 194.454 102.075) (width 1) (layer "B.Cu") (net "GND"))
 (segment (start 244.901 140.3015) (end 244.901 142.302) (width 1) (layer "B.Cu") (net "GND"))
 (segment (start 207.013 119.6545) (end 207.013 122.3485) (width 1) (layer "B.Cu") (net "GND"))
 (segment (start 225.089 88.6695) (end 222.394 91.3645) (width 1) (layer "B.Cu") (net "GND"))
 (segment (start 183.419 119.7925) (end 185.465 119.7925) (width 1) (layer "B.Cu") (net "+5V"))
 (segment (start 204.394 104.4385) (end 199.669 109.1635) (width 1) (layer "B.Cu") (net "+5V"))
 (segment (start 181.293 87.2925) (end 181.293 102.0275) (width 1) (layer "B.Cu") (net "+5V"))
 (segment (start 180.059 119.7925) (end 183.419 119.7925) (width 1) (layer "B.Cu") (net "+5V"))
 (segment (start 173.781 81.8815) (end 175.882 81.8815) (width 1) (layer "B.Cu") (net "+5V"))
 (segment (start 197.129 109.4335) (end 197.129 112.2265) (width 1) (layer "B.Cu") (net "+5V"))
 (segment (start 178.565 118.2985) (end 180.059 119.7925) (width 1) (layer "B.Cu") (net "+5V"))
 (segment (start 197.129 112.2265) (end 197.129 114.2125) (width 1) (layer "B.Cu") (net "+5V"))
 (segment (start 221.731 111.5755) (end 216.961 106.8055) (width 1) (layer "B.Cu") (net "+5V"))
 (segment (start 189.337572 129.588072) (end 192.669428 129.588072) (width 1) (layer "B.Cu") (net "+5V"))
 (segment (start 196.853 112.2265) (end 199.393 112.2265) (width 1) (layer "B.Cu") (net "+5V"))
 (segment (start 199.669 109.1635) (end 199.669 112.2265) (width 1) (layer "B.Cu") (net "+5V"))
 (segment (start 186.486 107.2205) (end 194.916 107.2205) (width 1) (layer "B.Cu") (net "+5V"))
 (segment (start 179.676 114.9525) (end 178.565 116.0635) (width 1) (layer "B.Cu") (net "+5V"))
 (segment (start 194.589 127.6685) (end 194.589 124.9265) (width 1) (layer "B.Cu") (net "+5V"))
 (segment (start 216.961 106.8055) (end 216.961 104.4385) (width 1) (layer "B.Cu") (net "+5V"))
 (segment (start 214.421 104.4385) (end 204.394 104.4385) (width 1) (layer "B.Cu") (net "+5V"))
 (segment (start 175.882 81.8815) (end 181.293 87.2925) (width 1) (layer "B.Cu") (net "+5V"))
 (segment (start 194.916 107.2205) (end 197.129 109.4335) (width 1) (layer "B.Cu") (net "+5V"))
 (segment (start 194.458 125.0715) (end 194.313 124.9265) (width 1) (layer "B.Cu") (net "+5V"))
 (segment (start 185.465 119.7925) (end 186.85 121.1775) (width 1) (layer "B.Cu") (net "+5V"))
 (segment (start 197.129 114.2125) (end 196.389 114.9525) (width 1) (layer "B.Cu") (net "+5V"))
 (segment (start 196.389 114.9525) (end 179.676 114.9525) (width 1) (layer "B.Cu") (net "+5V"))
 (segment (start 214.421 104.4385) (end 216.961 104.4385) (width 1) (layer "B.Cu") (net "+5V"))
 (segment (start 186.85 127.1005) (end 189.337572 129.588072) (width 1) (layer "B.Cu") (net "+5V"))
 (segment (start 178.565 116.0635) (end 178.565 118.2985) (width 1) (layer "B.Cu") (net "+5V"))
 (segment (start 186.85 121.1775) (end 186.85 127.1005) (width 1) (layer "B.Cu") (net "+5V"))
 (segment (start 229.587 111.5755) (end 221.731 111.5755) (width 1) (layer "B.Cu") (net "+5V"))
 (segment (start 181.293 102.0275) (end 186.486 107.2205) (width 1) (layer "B.Cu") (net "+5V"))
 (segment (start 192.669428 129.588072) (end 194.589 127.6685) (width 1) (layer "B.Cu") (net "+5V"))
 (segment (start 197.226 130.4165) (end 197.226 125.0235) (width 1) (layer "B.Cu") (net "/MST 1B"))
 (segment (start 197.226 125.0235) (end 197.129 124.9265) (width 1) (layer "B.Cu") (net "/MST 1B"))
 (segment (start 199.766 130.4165) (end 199.766 125.0235) (width 1) (layer "B.Cu") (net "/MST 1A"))
 (segment (start 199.766 125.0235) (end 199.669 124.9265) (width 1) (layer "B.Cu") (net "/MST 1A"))
 (segment (start 202.306 130.4165) (end 202.306 125.0235) (width 1) (layer "B.Cu") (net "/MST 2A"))
 (segment (start 202.306 125.0235) (end 202.209 124.9265) (width 1) (layer "B.Cu") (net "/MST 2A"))
 (segment (start 204.846 130.4165) (end 204.846 125.0235) (width 1) (layer "B.Cu") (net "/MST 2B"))
 (segment (start 204.846 125.0235) (end 204.749 124.9265) (width 1) (layer "B.Cu") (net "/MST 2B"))
 (segment (start 207.15 135.6545) (end 209.829 132.9755) (width 1) (layer "B.Cu") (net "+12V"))
 (segment (start 216.961 83.811) (end 216.961 85.8965) (width 1) (layer "B.Cu") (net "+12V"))
 (segment (start 204.185 94.6065) (end 207.8825 94.6065) (width 1) (layer "B.Cu") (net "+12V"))
 (segment (start 189.021 142.6615) (end 189.021 140.3015) (width 1) (layer "B.Cu") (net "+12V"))
 (segment (start 214.421 88.068) (end 214.421 85.8965) (width 1) (layer "B.Cu") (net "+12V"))
 (segment (start 189.538 96.206) (end 189.538 93.624) (width 1) (layer "B.Cu") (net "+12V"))
 (segment (start 201.1675 91.589) (end 204.185 94.6065) (width 1) (layer "B.Cu") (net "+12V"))
 (segment (start 222.2595 78.5125) (end 216.961 83.811) (width 1) (layer "B.Cu") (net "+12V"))
 (segment (start 192.8025 146.443) (end 189.021 142.6615) (width 1) (layer "B.Cu") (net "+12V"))
 (segment (start 189.021 140.3015) (end 189.021 137.2755) (width 1) (layer "B.Cu") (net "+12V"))
 (segment (start 189.021 137.2755) (end 190.642 135.6545) (width 1) (layer "B.Cu") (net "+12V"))
 (segment (start 232.201 137.1995) (end 232.201 140.3015) (width 1) (layer "B.Cu") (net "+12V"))
 (segment (start 189.538 93.624) (end 191.573 91.589) (width 1) (layer "B.Cu") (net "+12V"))
 (segment (start 246.736 134.6955) (end 234.705 134.6955) (width 1) (layer "B.Cu") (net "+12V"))
 (segment (start 190.642 135.6545) (end 207.15 135.6545) (width 1) (layer "B.Cu") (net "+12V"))
 (segment (start 248.524 132.9075) (end 248.524 78.5125) (width 1) (layer "B.Cu") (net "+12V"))
 (segment (start 248.524 132.9075) (end 246.736 134.6955) (width 1) (layer "B.Cu") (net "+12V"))
 (segment (start 207.8825 94.6065) (end 214.421 88.068) (width 1) (layer "B.Cu") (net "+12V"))
 (segment (start 244.9375 146.443) (end 192.8025 146.443) (width 1) (layer "B.Cu") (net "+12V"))
 (segment (start 191.573 91.589) (end 201.1675 91.589) (width 1) (layer "B.Cu") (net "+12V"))
 (segment (start 209.829 132.9755) (end 209.829 124.9265) (width 1) (layer "B.Cu") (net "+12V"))
 (segment (start 214.421 85.8965) (end 216.961 85.8965) (width 1) (layer "B.Cu") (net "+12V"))
 (segment (start 248.524 78.5125) (end 222.2595 78.5125) (width 1) (layer "B.Cu") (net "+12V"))
 (segment (start 248.524 142.8565) (end 244.9375 146.443) (width 1) (layer "B.Cu") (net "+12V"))
 (segment (start 234.705 134.6955) (end 232.201 137.1995) (width 1) (layer "B.Cu") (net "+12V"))
 (segment (start 248.524 132.9075) (end 248.524 142.8565) (width 1) (layer "B.Cu") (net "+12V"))
 (segment (start 193.9455 109.332) (end 194.589 109.9755) (width 1) (layer "B.Cu") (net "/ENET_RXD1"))
 (segment (start 194.589 109.9755) (end 194.589 112.2265) (width 1) (layer "B.Cu") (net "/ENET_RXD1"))
 (segment (start 179.467 105.6915) (end 183.1075 109.332) (width 1) (layer "B.Cu") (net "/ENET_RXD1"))
 (segment (start 179.467 88.44718) (end 179.467 105.6915) (width 1) (layer "B.Cu") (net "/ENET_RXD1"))
 (segment (start 183.1075 109.332) (end 193.9455 109.332) (width 1) (layer "B.Cu") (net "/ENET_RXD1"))
 (segment (start 173.781 84.4215) (end 175.44132 84.4215) (width 1) (layer "B.Cu") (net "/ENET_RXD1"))
 (segment (start 175.44132 84.4215) (end 179.467 88.44718) (width 1) (layer "B.Cu") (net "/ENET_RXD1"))
 (segment (start 173.827 84.4215) (end 173.923 84.5175) (width 1) (layer "B.Cu") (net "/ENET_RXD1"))
 (segment (start 173.781 84.4215) (end 173.827 84.4215) (width 1) (layer "B.Cu") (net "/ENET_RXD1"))
 (segment (start 177.685 88.7865) (end 177.685 107.4875) (width 1) (layer "B.Cu") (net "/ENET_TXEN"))
 (segment (start 177.685 107.4875) (end 182.424 112.2265) (width 1) (layer "B.Cu") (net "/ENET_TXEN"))
 (segment (start 175.86 86.9615) (end 177.685 88.7865) (width 1) (layer "B.Cu") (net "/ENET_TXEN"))
 (segment (start 173.781 86.9615) (end 175.86 86.9615) (width 1) (layer "B.Cu") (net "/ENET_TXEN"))
 (segment (start 182.424 112.2265) (end 192.049 112.2265) (width 1) (layer "B.Cu") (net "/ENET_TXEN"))
 (segment (start 183.419 122.3325) (end 181.289 122.3325) (width 1) (layer "B.Cu") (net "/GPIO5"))
 (segment (start 181.289 122.3325) (end 178.56 125.0615) (width 1) (layer "B.Cu") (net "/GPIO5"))
 (segment (start 178.56 125.0615) (end 173.781 125.0615) (width 1) (layer "B.Cu") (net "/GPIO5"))
 (segment (start 186.481 140.3015) (end 186.481 131.3155) (width 1) (layer "B.Cu") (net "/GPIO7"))
 (segment (start 182.767 127.6015) (end 173.781 127.6015) (width 1) (layer "B.Cu") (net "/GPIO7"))
 (segment (start 186.481 131.3155) (end 182.767 127.6015) (width 1) (layer "B.Cu") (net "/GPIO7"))
 (segment (start 182.671 130.1415) (end 173.781 130.1415) (width 1) (layer "B.Cu") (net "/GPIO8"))
 (segment (start 183.941 131.4115) (end 182.671 130.1415) (width 1) (layer "B.Cu") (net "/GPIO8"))
 (segment (start 183.941 140.3015) (end 183.941 131.4115) (width 1) (layer "B.Cu") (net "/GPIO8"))
 (segment (start 234.686 116.6555) (end 237.392 113.9495) (width 1) (layer "B.Cu") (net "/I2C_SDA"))
 (segment (start 237.392 113.9495) (end 237.392 108.0825) (width 1) (layer "B.Cu") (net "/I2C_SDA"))
 (segment (start 237.392 108.0825) (end 240.733 104.7415) (width 1) (layer "B.Cu") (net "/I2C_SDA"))
 (segment (start 229.587 116.6555) (end 234.686 116.6555) (width 1) (layer "B.Cu") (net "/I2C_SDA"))
 (segment (start 240.733 104.7415) (end 242.401 104.7415) (width 1) (layer "B.Cu") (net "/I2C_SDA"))
 (segment (start 240.31432 107.2815) (end 242.401 107.2815) (width 1) (layer "B.Cu") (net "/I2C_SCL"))
 (segment (start 239.202 114.8965) (end 239.202 108.39382) (width 1) (layer "B.Cu") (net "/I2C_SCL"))
 (segment (start 229.587 119.1955) (end 234.903 119.1955) (width 1) (layer "B.Cu") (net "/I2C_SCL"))
 (segment (start 239.202 108.39382) (end 240.31432 107.2815) (width 1) (layer "B.Cu") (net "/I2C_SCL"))
 (segment (start 234.903 119.1955) (end 239.202 114.8965) (width 1) (layer "B.Cu") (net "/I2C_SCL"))
 (segment (start 218.231 122.5215) (end 216.961 123.7915) (width 1) (layer "B.Cu") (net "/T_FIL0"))
 (segment (start 242.401 122.5215) (end 218.231 122.5215) (width 1) (layer "B.Cu") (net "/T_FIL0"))
 (segment (start 216.961 123.7915) (end 216.961 140.3015) (width 1) (layer "B.Cu") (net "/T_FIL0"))
 (segment (start 219.501 126.3315) (end 219.501 140.3015) (width 1) (layer "B.Cu") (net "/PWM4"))
 (segment (start 220.771 125.061499) (end 219.501 126.3315) (width 1) (layer "B.Cu") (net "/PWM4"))
 (segment (start 242.401 125.061499) (end 220.771 125.061499) (width 1) (layer "B.Cu") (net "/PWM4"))
 (segment (start 225.851 127.6015) (end 224.581 128.8715) (width 1) (layer "B.Cu") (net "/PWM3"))
 (segment (start 224.581 128.8715) (end 224.581 140.3015) (width 1) (layer "B.Cu") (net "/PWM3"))
 (segment (start 242.401 127.6015) (end 225.851 127.6015) (width 1) (layer "B.Cu") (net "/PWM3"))
 (segment (start 229.661 131.4115) (end 229.661 140.3015) (width 1) (layer "B.Cu") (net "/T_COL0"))
 (segment (start 242.401 130.1415) (end 230.931 130.1415) (width 1) (layer "B.Cu") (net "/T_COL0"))
 (segment (start 230.931 130.1415) (end 229.661 131.4115) (width 1) (layer "B.Cu") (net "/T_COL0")))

